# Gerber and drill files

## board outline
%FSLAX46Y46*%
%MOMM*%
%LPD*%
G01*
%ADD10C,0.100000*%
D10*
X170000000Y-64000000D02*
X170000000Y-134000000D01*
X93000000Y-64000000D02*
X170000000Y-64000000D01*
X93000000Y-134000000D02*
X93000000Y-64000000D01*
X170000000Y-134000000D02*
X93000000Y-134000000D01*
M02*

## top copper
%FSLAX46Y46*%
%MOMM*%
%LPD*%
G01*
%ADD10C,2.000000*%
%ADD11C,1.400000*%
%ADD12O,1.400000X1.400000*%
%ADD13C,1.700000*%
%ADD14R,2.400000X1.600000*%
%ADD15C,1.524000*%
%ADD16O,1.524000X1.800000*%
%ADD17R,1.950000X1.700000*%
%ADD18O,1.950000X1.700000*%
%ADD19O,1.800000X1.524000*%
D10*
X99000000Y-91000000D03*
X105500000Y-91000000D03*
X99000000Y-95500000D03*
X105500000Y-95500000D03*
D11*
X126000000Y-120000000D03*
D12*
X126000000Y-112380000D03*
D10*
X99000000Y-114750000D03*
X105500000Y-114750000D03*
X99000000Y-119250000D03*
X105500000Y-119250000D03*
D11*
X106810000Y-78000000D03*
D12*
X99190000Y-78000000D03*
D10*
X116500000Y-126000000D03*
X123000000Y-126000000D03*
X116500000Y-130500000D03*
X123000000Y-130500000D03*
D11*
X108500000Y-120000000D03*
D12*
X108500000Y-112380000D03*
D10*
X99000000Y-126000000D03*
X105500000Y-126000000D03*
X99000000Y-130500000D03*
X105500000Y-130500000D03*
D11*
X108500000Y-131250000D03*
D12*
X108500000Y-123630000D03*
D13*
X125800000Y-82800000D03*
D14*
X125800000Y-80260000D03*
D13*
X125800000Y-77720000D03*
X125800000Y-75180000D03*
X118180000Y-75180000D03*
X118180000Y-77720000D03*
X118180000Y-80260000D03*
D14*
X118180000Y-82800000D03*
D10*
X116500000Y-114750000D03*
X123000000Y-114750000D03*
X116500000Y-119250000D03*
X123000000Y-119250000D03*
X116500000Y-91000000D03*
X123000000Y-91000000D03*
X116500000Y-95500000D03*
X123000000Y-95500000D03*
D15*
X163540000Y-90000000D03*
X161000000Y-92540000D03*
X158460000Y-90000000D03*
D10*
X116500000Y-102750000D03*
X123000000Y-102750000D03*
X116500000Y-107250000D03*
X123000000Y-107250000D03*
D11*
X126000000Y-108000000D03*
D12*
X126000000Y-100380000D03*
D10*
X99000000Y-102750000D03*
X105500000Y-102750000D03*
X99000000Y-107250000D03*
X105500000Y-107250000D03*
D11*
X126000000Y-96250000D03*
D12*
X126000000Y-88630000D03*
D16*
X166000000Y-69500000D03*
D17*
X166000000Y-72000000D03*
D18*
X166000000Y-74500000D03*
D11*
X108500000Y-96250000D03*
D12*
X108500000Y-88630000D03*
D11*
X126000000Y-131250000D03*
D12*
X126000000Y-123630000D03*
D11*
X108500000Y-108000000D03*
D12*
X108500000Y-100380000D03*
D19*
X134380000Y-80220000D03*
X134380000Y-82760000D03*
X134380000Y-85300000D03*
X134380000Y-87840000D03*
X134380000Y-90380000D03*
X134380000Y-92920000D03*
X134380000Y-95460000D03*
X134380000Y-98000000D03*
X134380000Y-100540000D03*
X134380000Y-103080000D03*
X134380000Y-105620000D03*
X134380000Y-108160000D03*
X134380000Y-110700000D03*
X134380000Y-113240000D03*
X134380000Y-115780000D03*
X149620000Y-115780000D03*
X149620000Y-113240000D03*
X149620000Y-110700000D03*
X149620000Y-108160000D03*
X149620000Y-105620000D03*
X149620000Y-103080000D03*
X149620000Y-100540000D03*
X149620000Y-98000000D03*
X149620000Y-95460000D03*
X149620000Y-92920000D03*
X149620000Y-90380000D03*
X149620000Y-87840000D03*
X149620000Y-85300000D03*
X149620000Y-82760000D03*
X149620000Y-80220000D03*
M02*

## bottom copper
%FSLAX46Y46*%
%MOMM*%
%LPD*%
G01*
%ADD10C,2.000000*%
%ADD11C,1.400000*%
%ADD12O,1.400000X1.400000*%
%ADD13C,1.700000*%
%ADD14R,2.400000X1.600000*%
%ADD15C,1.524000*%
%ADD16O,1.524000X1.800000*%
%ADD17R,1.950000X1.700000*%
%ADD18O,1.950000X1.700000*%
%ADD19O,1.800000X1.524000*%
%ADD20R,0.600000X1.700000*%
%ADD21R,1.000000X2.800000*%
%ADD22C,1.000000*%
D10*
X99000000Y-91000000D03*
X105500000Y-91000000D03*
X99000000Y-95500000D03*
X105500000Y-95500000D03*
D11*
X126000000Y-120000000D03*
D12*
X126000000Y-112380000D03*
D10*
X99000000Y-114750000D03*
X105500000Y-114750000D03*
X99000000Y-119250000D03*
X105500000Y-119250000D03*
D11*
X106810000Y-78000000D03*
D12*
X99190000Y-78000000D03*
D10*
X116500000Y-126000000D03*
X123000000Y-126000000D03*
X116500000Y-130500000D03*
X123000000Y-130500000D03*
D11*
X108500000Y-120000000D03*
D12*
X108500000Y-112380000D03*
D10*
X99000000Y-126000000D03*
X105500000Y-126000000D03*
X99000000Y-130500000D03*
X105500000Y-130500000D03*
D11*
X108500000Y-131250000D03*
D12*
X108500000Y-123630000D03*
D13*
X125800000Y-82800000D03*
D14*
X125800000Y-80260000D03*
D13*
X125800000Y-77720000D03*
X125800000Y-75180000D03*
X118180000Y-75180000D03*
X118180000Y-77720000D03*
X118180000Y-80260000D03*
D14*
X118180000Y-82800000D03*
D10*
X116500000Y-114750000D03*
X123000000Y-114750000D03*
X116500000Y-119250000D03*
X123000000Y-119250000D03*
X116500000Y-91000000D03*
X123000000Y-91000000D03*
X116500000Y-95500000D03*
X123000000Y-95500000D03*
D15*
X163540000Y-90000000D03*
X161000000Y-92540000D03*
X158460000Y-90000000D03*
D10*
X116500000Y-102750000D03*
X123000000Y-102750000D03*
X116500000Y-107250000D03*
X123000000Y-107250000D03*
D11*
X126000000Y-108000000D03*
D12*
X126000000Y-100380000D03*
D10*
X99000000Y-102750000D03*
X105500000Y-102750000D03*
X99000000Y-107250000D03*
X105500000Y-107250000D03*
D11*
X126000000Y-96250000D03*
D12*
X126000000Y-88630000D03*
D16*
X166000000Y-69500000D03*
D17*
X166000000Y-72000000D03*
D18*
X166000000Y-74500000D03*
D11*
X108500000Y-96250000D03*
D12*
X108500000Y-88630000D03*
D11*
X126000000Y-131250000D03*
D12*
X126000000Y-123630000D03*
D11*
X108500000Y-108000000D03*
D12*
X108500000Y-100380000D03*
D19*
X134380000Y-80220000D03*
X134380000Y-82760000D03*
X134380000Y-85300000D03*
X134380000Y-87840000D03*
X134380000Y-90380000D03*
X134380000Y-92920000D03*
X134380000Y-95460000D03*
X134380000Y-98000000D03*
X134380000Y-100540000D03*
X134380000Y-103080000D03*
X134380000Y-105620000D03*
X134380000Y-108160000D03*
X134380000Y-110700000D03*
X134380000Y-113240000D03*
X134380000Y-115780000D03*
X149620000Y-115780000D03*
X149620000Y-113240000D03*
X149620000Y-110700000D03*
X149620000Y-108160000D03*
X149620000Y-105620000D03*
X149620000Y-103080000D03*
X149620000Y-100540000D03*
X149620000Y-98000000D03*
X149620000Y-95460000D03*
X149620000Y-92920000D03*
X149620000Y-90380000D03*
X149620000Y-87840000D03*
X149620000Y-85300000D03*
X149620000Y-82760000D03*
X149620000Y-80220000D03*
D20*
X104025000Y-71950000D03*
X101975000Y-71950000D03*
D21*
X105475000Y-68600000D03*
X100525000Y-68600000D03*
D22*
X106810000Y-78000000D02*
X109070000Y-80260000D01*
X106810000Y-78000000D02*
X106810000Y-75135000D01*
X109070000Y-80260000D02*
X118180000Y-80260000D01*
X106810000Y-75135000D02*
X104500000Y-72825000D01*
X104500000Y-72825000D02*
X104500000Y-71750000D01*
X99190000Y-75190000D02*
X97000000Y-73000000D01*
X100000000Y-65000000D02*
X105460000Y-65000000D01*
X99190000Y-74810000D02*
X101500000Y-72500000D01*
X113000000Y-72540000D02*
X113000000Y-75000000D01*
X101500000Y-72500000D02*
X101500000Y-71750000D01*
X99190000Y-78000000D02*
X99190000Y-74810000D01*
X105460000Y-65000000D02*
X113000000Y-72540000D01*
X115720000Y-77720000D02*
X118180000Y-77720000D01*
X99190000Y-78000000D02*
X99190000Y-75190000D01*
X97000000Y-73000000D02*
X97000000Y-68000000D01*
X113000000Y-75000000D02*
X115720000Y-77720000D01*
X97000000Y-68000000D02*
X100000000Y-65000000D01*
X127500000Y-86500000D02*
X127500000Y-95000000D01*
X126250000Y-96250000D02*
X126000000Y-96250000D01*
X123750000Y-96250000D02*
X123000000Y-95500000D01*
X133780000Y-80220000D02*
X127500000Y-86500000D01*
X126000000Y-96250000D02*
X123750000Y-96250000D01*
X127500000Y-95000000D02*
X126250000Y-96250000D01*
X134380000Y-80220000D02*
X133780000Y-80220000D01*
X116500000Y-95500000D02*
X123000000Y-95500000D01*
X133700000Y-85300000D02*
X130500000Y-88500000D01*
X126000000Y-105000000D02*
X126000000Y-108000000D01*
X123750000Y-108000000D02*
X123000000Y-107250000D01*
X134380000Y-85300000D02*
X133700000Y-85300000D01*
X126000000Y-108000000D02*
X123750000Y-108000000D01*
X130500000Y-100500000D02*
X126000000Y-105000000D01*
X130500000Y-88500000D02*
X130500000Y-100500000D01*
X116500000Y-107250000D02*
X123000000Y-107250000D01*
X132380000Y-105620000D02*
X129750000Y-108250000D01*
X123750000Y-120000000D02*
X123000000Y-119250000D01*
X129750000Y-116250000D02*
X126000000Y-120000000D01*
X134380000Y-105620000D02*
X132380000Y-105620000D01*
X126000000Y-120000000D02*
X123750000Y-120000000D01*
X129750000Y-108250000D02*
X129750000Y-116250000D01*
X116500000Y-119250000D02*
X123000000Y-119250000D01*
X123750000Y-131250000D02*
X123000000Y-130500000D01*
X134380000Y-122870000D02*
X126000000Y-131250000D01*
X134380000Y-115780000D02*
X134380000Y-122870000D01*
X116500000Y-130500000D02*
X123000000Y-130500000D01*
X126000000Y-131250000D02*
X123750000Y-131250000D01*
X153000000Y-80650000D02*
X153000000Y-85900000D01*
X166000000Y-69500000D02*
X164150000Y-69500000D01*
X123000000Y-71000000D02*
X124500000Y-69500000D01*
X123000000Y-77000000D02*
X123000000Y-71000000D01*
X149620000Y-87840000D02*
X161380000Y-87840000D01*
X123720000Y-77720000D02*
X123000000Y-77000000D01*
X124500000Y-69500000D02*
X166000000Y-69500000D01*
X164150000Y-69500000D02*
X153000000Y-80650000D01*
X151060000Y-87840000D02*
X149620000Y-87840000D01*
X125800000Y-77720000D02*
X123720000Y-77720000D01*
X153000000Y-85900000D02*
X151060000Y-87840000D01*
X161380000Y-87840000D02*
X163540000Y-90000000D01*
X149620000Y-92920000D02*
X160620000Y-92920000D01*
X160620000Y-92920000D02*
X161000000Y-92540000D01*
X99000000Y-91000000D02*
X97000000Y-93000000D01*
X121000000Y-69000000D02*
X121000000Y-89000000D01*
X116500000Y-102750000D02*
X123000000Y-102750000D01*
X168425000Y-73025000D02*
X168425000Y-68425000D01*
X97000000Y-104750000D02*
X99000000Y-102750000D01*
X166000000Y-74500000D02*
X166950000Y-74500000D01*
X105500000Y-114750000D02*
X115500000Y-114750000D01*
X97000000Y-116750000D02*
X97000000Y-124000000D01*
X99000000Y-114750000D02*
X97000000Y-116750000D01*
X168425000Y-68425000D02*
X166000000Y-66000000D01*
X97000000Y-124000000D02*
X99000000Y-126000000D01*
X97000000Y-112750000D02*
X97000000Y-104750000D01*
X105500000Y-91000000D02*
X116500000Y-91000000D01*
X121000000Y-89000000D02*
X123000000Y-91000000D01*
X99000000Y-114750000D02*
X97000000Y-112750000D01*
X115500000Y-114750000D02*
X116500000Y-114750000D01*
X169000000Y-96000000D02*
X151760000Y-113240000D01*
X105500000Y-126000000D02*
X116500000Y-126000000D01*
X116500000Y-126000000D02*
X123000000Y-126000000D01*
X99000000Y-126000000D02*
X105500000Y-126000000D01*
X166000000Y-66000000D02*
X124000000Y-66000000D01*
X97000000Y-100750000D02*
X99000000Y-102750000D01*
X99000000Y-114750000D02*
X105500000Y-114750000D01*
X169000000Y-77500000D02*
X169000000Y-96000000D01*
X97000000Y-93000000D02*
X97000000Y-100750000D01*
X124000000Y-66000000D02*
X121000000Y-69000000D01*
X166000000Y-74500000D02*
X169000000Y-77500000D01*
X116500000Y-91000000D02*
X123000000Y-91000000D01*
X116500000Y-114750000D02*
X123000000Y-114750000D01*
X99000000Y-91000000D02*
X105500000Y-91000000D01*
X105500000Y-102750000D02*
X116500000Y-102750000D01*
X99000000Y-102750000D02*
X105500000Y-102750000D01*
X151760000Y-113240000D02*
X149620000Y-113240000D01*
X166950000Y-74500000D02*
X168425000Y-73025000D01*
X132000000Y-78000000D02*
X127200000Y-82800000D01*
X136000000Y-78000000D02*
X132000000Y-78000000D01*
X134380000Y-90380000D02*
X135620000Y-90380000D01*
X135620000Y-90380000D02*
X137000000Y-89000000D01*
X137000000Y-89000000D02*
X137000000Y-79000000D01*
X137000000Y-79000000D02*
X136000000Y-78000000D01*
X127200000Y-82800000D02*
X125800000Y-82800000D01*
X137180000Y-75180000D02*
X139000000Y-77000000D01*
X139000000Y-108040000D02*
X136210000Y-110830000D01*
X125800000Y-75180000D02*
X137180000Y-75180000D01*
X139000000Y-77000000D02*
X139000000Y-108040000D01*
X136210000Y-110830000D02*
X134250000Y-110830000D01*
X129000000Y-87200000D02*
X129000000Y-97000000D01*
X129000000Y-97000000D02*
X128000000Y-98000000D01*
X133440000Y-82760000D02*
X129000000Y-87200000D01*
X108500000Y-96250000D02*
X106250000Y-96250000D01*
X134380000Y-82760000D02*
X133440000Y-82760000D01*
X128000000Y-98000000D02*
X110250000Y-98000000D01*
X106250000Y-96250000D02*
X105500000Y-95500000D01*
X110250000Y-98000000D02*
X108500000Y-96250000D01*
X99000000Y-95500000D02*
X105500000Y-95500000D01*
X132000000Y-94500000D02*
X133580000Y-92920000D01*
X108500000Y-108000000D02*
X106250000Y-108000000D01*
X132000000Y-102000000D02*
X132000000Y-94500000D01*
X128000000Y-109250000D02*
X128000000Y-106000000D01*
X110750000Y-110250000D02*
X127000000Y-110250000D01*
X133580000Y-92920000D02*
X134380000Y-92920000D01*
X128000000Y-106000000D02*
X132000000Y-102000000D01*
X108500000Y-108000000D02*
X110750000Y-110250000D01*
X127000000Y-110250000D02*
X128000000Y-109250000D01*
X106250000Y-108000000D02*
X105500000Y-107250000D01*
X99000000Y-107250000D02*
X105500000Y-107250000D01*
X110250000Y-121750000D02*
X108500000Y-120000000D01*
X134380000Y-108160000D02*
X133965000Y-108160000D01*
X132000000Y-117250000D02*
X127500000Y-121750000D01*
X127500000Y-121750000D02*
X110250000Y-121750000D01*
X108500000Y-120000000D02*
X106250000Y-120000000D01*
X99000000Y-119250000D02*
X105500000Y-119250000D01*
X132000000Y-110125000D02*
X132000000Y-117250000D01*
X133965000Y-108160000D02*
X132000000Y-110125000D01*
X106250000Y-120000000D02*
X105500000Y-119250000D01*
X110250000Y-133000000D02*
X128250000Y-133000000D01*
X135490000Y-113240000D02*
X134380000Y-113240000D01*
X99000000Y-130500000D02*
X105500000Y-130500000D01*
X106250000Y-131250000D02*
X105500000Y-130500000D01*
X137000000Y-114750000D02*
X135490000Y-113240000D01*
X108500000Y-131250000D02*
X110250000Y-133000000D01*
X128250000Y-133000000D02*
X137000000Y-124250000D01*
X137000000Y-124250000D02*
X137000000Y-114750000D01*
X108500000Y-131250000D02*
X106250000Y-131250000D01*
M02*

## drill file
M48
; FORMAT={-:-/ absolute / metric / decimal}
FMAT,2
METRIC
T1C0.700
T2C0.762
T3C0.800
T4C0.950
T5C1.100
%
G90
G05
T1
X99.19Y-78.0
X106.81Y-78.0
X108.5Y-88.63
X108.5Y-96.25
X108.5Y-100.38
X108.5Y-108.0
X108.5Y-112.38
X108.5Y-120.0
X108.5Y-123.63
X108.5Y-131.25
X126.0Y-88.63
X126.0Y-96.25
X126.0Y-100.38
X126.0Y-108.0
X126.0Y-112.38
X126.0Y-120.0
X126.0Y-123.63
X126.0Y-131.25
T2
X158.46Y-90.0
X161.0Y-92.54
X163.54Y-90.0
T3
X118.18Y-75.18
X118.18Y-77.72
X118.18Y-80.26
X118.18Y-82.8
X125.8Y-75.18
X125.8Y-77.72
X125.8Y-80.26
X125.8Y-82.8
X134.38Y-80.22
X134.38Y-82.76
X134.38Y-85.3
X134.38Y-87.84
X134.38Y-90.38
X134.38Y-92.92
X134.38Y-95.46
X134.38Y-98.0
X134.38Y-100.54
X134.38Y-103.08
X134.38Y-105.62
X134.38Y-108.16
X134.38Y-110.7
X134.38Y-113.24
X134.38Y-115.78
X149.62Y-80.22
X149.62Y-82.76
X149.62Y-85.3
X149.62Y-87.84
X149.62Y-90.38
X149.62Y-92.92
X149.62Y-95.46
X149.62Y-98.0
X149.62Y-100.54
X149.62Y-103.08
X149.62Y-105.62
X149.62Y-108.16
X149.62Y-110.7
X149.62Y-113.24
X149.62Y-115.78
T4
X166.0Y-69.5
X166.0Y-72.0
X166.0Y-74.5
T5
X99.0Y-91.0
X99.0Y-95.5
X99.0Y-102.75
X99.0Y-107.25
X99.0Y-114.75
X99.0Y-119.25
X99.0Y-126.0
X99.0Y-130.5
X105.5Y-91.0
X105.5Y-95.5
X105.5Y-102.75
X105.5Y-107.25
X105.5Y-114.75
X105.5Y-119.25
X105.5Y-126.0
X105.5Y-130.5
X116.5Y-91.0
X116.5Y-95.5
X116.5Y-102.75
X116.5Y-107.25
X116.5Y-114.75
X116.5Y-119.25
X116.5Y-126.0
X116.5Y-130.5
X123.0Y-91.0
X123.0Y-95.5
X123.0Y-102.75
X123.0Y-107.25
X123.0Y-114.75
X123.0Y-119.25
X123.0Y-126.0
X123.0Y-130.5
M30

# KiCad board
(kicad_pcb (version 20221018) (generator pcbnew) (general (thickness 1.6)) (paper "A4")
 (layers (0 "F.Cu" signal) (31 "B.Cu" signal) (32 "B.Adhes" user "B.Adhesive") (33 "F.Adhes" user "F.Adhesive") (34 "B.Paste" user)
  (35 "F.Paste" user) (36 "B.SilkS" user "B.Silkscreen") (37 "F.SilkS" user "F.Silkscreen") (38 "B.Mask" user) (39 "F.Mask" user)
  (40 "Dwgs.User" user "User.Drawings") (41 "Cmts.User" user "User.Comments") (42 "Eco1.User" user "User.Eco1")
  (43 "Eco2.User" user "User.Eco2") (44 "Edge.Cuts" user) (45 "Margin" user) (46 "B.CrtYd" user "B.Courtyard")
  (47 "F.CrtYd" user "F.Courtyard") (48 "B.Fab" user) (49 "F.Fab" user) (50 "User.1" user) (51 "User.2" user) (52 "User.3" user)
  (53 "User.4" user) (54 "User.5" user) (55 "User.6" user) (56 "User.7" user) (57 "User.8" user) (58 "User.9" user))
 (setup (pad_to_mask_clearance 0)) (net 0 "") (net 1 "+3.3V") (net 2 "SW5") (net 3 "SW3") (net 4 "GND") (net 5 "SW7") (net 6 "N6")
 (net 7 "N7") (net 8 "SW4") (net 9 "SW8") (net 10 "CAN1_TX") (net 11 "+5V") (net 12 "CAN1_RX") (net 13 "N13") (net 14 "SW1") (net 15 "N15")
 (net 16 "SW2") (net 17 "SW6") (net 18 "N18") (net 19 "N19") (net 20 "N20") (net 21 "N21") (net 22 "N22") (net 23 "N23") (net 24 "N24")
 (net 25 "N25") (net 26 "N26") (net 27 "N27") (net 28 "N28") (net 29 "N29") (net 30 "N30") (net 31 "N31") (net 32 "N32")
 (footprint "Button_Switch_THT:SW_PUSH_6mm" (layer "F.Cu") (at 99 91)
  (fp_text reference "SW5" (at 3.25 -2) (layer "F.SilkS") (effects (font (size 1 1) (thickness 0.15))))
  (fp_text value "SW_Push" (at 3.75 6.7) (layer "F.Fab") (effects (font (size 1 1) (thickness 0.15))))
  (pad "1" thru_hole circle (at 0 0 90) (size 2 2) (drill 1.1) (layers "*.Cu" "*.Mask") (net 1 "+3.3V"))
  (pad "1" thru_hole circle (at 6.5 0 90) (size 2 2) (drill 1.1) (layers "*.Cu" "*.Mask") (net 1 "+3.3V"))
  (pad "2" thru_hole circle (at 0 4.5 90) (size 2 2) (drill 1.1) (layers "*.Cu" "*.Mask") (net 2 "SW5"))
  (pad "2" thru_hole circle (at 6.5 4.5 90) (size 2 2) (drill 1.1) (layers "*.Cu" "*.Mask") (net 2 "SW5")))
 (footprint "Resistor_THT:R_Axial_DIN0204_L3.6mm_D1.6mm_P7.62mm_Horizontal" (layer "F.Cu") (at 126 120 90)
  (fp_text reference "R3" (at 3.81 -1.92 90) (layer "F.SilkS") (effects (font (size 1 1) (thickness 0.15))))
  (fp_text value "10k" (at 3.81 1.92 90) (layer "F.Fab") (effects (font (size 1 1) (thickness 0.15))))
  (pad "1" thru_hole circle (at 0 0 90) (size 1.4 1.4) (drill 0.7) (layers "*.Cu" "*.Mask") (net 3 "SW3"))
  (pad "2" thru_hole oval (at 7.62 0 90) (size 1.4 1.4) (drill 0.7) (layers "*.Cu" "*.Mask") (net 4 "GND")))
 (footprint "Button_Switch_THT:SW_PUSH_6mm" (layer "F.Cu") (at 99 114.75)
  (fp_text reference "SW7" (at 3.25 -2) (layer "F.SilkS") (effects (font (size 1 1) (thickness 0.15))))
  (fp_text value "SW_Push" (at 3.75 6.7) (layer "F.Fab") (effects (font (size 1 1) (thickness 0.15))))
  (pad "1" thru_hole circle (at 0 0 90) (size 2 2) (drill 1.1) (layers "*.Cu" "*.Mask") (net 1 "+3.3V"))
  (pad "1" thru_hole circle (at 6.5 0 90) (size 2 2) (drill 1.1) (layers "*.Cu" "*.Mask") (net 1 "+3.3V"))
  (pad "2" thru_hole circle (at 0 4.5 90) (size 2 2) (drill 1.1) (layers "*.Cu" "*.Mask") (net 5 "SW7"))
  (pad "2" thru_hole circle (at 6.5 4.5 90) (size 2 2) (drill 1.1) (layers "*.Cu" "*.Mask") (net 5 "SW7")))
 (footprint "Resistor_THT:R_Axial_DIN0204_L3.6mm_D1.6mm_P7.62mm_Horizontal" (layer "F.Cu") (at 106.81 78 180)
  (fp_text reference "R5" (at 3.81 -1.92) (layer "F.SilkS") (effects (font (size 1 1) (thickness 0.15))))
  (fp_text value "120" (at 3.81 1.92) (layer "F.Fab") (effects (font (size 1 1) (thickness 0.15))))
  (pad "1" thru_hole circle (at 0 0 180) (size 1.4 1.4) (drill 0.7) (layers "*.Cu" "*.Mask") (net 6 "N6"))
  (pad "2" thru_hole oval (at 7.62 0 180) (size 1.4 1.4) (drill 0.7) (layers "*.Cu" "*.Mask") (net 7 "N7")))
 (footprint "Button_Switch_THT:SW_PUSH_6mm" (layer "F.Cu") (at 116.5 126)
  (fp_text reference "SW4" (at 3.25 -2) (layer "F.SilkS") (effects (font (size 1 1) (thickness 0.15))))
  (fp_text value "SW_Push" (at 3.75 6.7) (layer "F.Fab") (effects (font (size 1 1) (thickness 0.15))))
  (pad "1" thru_hole circle (at 0 0 90) (size 2 2) (drill 1.1) (layers "*.Cu" "*.Mask") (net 1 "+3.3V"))
  (pad "1" thru_hole circle (at 6.5 0 90) (size 2 2) (drill 1.1) (layers "*.Cu" "*.Mask") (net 1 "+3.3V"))
  (pad "2" thru_hole circle (at 0 4.5 90) (size 2 2) (drill 1.1) (layers "*.Cu" "*.Mask") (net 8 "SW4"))
  (pad "2" thru_hole circle (at 6.5 4.5 90) (size 2 2) (drill 1.1) (layers "*.Cu" "*.Mask") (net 8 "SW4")))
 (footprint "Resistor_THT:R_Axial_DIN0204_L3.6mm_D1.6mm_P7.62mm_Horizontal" (layer "F.Cu") (at 108.5 120 90)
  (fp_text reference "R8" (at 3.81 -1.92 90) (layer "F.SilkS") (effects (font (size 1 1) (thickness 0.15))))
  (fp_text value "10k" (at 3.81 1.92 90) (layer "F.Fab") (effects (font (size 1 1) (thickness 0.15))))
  (pad "1" thru_hole circle (at 0 0 90) (size 1.4 1.4) (drill 0.7) (layers "*.Cu" "*.Mask") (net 5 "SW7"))
  (pad "2" thru_hole oval (at 7.62 0 90) (size 1.4 1.4) (drill 0.7) (layers "*.Cu" "*.Mask") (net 4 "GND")))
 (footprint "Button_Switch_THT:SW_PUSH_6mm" (layer "F.Cu") (at 99 126)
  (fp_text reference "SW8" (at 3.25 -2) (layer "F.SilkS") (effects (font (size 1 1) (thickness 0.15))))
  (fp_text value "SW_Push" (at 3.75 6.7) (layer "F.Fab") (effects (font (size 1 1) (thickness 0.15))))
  (pad "1" thru_hole circle (at 0 0 90) (size 2 2) (drill 1.1) (layers "*.Cu" "*.Mask") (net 1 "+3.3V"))
  (pad "1" thru_hole circle (at 6.5 0 90) (size 2 2) (drill 1.1) (layers "*.Cu" "*.Mask") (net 1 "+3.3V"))
  (pad "2" thru_hole circle (at 0 4.5 90) (size 2 2) (drill 1.1) (layers "*.Cu" "*.Mask") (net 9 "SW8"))
  (pad "2" thru_hole circle (at 6.5 4.5 90) (size 2 2) (drill 1.1) (layers "*.Cu" "*.Mask") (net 9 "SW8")))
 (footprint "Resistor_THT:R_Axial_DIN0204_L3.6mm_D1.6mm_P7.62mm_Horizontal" (layer "F.Cu") (at 108.5 131.25 90)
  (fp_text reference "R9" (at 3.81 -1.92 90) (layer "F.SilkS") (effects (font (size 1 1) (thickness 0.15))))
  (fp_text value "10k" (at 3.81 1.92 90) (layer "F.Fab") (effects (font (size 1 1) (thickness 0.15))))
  (pad "1" thru_hole circle (at 0 0 90) (size 1.4 1.4) (drill 0.7) (layers "*.Cu" "*.Mask") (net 9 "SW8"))
  (pad "2" thru_hole oval (at 7.62 0 90) (size 1.4 1.4) (drill 0.7) (layers "*.Cu" "*.Mask") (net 4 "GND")))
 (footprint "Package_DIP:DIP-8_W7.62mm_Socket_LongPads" (layer "F.Cu") (at 125.8 82.8 180)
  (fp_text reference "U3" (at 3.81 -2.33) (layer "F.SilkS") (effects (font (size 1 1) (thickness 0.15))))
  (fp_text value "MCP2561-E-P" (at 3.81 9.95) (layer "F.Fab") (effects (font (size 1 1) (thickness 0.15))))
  (pad "1" thru_hole circle (at 0 0 180) (size 1.7 1.7) (drill 0.8) (layers "*.Cu" "*.Mask") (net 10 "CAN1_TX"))
  (pad "2" thru_hole rect (at 0 2.54 180) (size 2.4 1.6) (drill 0.8) (layers "*.Cu" "*.Mask") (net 4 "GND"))
  (pad "3" thru_hole circle (at 0 5.08 180) (size 1.7 1.7) (drill 0.8) (layers "*.Cu" "*.Mask") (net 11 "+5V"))
  (pad "4" thru_hole circle (at 0 7.62 180) (size 1.7 1.7) (drill 0.8) (layers "*.Cu" "*.Mask") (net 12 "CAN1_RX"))
  (pad "5" thru_hole circle (at 7.62 7.62 180) (size 1.7 1.7) (drill 0.8) (layers "*.Cu" "*.Mask") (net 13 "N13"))
  (pad "6" thru_hole circle (at 7.62 5.08 180) (size 1.7 1.7) (drill 0.8) (layers "*.Cu" "*.Mask") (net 7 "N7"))
  (pad "7" thru_hole circle (at 7.62 2.54 180) (size 1.7 1.7) (drill 0.8) (layers "*.Cu" "*.Mask") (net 6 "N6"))
  (pad "8" thru_hole rect (at 7.62 0 180) (size 2.4 1.6) (drill 0.8) (layers "*.Cu" "*.Mask") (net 4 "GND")))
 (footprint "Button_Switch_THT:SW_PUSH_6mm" (layer "F.Cu") (at 116.5 114.75)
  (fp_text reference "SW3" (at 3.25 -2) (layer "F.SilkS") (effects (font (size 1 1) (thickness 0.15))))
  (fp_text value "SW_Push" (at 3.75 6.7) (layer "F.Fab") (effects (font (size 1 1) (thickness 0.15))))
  (pad "1" thru_hole circle (at 0 0 90) (size 2 2) (drill 1.1) (layers "*.Cu" "*.Mask") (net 1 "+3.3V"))
  (pad "1" thru_hole circle (at 6.5 0 90) (size 2 2) (drill 1.1) (layers "*.Cu" "*.Mask") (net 1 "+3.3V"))
  (pad "2" thru_hole circle (at 0 4.5 90) (size 2 2) (drill 1.1) (layers "*.Cu" "*.Mask") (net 3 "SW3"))
  (pad "2" thru_hole circle (at 6.5 4.5 90) (size 2 2) (drill 1.1) (layers "*.Cu" "*.Mask") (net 3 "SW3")))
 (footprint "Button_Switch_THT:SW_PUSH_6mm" (layer "F.Cu") (at 116.5 91)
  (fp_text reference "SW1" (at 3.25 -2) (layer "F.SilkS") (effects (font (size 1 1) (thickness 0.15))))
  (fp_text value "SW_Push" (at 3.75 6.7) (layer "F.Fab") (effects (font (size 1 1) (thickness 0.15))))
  (pad "1" thru_hole circle (at 0 0 90) (size 2 2) (drill 1.1) (layers "*.Cu" "*.Mask") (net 1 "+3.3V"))
  (pad "1" thru_hole circle (at 6.5 0 90) (size 2 2) (drill 1.1) (layers "*.Cu" "*.Mask") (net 1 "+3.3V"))
  (pad "2" thru_hole circle (at 0 4.5 90) (size 2 2) (drill 1.1) (layers "*.Cu" "*.Mask") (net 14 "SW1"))
  (pad "2" thru_hole circle (at 6.5 4.5 90) (size 2 2) (drill 1.1) (layers "*.Cu" "*.Mask") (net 14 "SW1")))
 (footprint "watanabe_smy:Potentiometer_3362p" (layer "F.Cu") (at 161 90 180)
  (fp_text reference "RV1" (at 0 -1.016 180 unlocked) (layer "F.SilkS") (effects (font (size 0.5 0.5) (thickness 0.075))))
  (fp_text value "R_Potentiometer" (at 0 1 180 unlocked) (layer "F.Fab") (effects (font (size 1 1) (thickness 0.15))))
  (pad "1" thru_hole circle (at -2.54 0 180) (size 1.524 1.524) (drill 0.762) (layers "*.Cu" "*.Mask") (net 11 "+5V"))
  (pad "2" thru_hole circle (at 0 -2.54 180) (size 1.524 1.524) (drill 0.762) (layers "*.Cu" "*.Mask") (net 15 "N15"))
  (pad "3" thru_hole circle (at 2.54 0 180) (size 1.524 1.524) (drill 0.762) (layers "*.Cu" "*.Mask") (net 4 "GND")))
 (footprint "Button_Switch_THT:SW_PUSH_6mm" (layer "F.Cu") (at 116.5 102.75)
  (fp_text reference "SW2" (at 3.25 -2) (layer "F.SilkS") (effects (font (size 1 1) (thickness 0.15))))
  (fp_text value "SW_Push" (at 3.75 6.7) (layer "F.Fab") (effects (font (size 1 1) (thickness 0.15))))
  (pad "1" thru_hole circle (at 0 0 90) (size 2 2) (drill 1.1) (layers "*.Cu" "*.Mask") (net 1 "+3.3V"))
  (pad "1" thru_hole circle (at 6.5 0 90) (size 2 2) (drill 1.1) (layers "*.Cu" "*.Mask") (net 1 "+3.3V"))
  (pad "2" thru_hole circle (at 0 4.5 90) (size 2 2) (drill 1.1) (layers "*.Cu" "*.Mask") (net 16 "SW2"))
  (pad "2" thru_hole circle (at 6.5 4.5 90) (size 2 2) (drill 1.1) (layers "*.Cu" "*.Mask") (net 16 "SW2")))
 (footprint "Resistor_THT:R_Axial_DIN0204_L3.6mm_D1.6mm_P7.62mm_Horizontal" (layer "F.Cu") (at 126 108 90)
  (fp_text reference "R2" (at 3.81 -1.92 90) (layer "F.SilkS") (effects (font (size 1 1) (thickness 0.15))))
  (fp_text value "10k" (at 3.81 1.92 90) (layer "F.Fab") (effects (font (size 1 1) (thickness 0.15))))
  (pad "1" thru_hole circle (at 0 0 90) (size 1.4 1.4) (drill 0.7) (layers "*.Cu" "*.Mask") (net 16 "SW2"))
  (pad "2" thru_hole oval (at 7.62 0 90) (size 1.4 1.4) (drill 0.7) (layers "*.Cu" "*.Mask") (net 4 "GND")))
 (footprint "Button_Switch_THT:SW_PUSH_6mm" (layer "F.Cu") (at 99 102.75)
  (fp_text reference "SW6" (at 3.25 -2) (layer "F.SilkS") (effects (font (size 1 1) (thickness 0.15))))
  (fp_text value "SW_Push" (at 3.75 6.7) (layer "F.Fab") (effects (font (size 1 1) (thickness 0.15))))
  (pad "1" thru_hole circle (at 0 0 90) (size 2 2) (drill 1.1) (layers "*.Cu" "*.Mask") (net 1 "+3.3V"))
  (pad "1" thru_hole circle (at 6.5 0 90) (size 2 2) (drill 1.1) (layers "*.Cu" "*.Mask") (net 1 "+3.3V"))
  (pad "2" thru_hole circle (at 0 4.5 90) (size 2 2) (drill 1.1) (layers "*.Cu" "*.Mask") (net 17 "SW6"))
  (pad "2" thru_hole circle (at 6.5 4.5 90) (size 2 2) (drill 1.1) (layers "*.Cu" "*.Mask") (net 17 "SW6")))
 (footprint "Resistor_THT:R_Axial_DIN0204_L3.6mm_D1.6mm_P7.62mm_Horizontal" (layer "F.Cu") (at 126 96.25 90)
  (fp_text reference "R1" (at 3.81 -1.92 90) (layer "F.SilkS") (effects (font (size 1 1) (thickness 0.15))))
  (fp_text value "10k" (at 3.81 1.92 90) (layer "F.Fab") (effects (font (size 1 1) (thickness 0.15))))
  (pad "1" thru_hole circle (at 0 0 90) (size 1.4 1.4) (drill 0.7) (layers "*.Cu" "*.Mask") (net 14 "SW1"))
  (pad "2" thru_hole oval (at 7.62 0 90) (size 1.4 1.4) (drill 0.7) (layers "*.Cu" "*.Mask") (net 4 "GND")))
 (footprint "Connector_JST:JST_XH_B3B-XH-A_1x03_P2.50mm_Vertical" (layer "F.Cu") (at 166 69.5 -90)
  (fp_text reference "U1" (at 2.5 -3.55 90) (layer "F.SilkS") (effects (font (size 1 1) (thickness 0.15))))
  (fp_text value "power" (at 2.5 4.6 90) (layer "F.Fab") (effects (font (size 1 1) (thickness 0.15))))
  (pad "1" thru_hole oval (at 0 0 270) (size 1.8 1.524) (drill 0.95) (layers "*.Cu" "*.Mask") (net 11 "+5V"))
  (pad "2" thru_hole rect (at 2.5 0 270) (size 1.7 1.95) (drill 0.95) (layers "*.Cu" "*.Mask") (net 4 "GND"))
  (pad "3" thru_hole oval (at 5 0 270) (size 1.7 1.95) (drill 0.95) (layers "*.Cu" "*.Mask") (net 1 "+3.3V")))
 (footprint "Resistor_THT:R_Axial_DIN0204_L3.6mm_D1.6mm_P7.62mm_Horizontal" (layer "F.Cu") (at 108.5 96.25 90)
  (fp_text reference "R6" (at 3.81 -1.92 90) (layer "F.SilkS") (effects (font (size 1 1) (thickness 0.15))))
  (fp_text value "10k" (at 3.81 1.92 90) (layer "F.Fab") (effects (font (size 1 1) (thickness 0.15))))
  (pad "1" thru_hole circle (at 0 0 90) (size 1.4 1.4) (drill 0.7) (layers "*.Cu" "*.Mask") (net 2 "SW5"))
  (pad "2" thru_hole oval (at 7.62 0 90) (size 1.4 1.4) (drill 0.7) (layers "*.Cu" "*.Mask") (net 4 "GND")))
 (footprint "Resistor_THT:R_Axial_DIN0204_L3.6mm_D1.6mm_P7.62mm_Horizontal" (layer "F.Cu") (at 126 131.25 90)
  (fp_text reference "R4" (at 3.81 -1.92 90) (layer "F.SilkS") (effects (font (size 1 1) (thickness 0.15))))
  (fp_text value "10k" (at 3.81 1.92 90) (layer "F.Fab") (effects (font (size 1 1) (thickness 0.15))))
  (pad "1" thru_hole circle (at 0 0 90) (size 1.4 1.4) (drill 0.7) (layers "*.Cu" "*.Mask") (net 8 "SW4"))
  (pad "2" thru_hole oval (at 7.62 0 90) (size 1.4 1.4) (drill 0.7) (layers "*.Cu" "*.Mask") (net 4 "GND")))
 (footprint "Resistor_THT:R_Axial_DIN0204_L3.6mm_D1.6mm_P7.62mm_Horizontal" (layer "F.Cu") (at 108.5 108 90)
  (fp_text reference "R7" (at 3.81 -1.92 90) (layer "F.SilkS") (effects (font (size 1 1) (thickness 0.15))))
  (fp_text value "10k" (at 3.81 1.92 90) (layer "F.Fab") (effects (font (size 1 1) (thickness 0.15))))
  (pad "1" thru_hole circle (at 0 0 90) (size 1.4 1.4) (drill 0.7) (layers "*.Cu" "*.Mask") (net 17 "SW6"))
  (pad "2" thru_hole oval (at 7.62 0 90) (size 1.4 1.4) (drill 0.7) (layers "*.Cu" "*.Mask") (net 4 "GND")))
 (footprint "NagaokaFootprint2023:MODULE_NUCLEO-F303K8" (layer "F.Cu") (at 142 98)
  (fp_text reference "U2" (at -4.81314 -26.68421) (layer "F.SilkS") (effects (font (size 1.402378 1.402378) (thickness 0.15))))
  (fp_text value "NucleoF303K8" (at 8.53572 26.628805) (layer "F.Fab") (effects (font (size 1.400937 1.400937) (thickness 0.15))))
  (pad "1" thru_hole oval (at -7.62 -17.78) (size 1.8 1.524) (drill 0.8) (layers "*.Cu" "*.Mask") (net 14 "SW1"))
  (pad "2" thru_hole oval (at -7.62 -15.24) (size 1.8 1.524) (drill 0.8) (layers "*.Cu" "*.Mask") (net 2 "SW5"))
  (pad "3" thru_hole oval (at -7.62 -12.7) (size 1.8 1.524) (drill 0.8) (layers "*.Cu" "*.Mask") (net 16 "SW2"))
  (pad "4" thru_hole oval (at -7.62 -10.16) (size 1.8 1.524) (drill 0.8) (layers "*.Cu" "*.Mask") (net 4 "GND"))
  (pad "5" thru_hole oval (at -7.62 -7.62) (size 1.8 1.524) (drill 0.8) (layers "*.Cu" "*.Mask") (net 10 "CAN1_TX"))
  (pad "6" thru_hole oval (at -7.62 -5.08) (size 1.8 1.524) (drill 0.8) (layers "*.Cu" "*.Mask") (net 17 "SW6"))
  (pad "7" thru_hole oval (at -7.62 -2.54) (size 1.8 1.524) (drill 0.8) (layers "*.Cu" "*.Mask") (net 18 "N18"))
  (pad "8" thru_hole oval (at -7.62 0) (size 1.8 1.524) (drill 0.8) (layers "*.Cu" "*.Mask") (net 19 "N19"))
  (pad "9" thru_hole oval (at -7.62 2.54) (size 1.8 1.524) (drill 0.8) (layers "*.Cu" "*.Mask") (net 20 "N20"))
  (pad "10" thru_hole oval (at -7.62 5.08) (size 1.8 1.524) (drill 0.8) (layers "*.Cu" "*.Mask") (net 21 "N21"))
  (pad "11" thru_hole oval (at -7.62 7.62) (size 1.8 1.524) (drill 0.8) (layers "*.Cu" "*.Mask") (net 3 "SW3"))
  (pad "12" thru_hole oval (at -7.62 10.16) (size 1.8 1.524) (drill 0.8) (layers "*.Cu" "*.Mask") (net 5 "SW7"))
  (pad "13" thru_hole oval (at -7.62 12.7) (size 1.8 1.524) (drill 0.8) (layers "*.Cu" "*.Mask") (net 12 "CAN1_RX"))
  (pad "14" thru_hole oval (at -7.62 15.24) (size 1.8 1.524) (drill 0.8) (layers "*.Cu" "*.Mask") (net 9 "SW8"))
  (pad "15" thru_hole oval (at -7.62 17.78) (size 1.8 1.524) (drill 0.8) (layers "*.Cu" "*.Mask") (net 8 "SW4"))
  (pad "16" thru_hole oval (at 7.62 17.78) (size 1.8 1.524) (drill 0.8) (layers "*.Cu" "*.Mask") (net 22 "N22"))
  (pad "17" thru_hole oval (at 7.62 15.24) (size 1.8 1.524) (drill 0.8) (layers "*.Cu" "*.Mask") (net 1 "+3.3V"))
  (pad "18" thru_hole oval (at 7.62 12.7) (size 1.8 1.524) (drill 0.8) (layers "*.Cu" "*.Mask") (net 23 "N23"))
  (pad "19" thru_hole oval (at 7.62 10.16) (size 1.8 1.524) (drill 0.8) (layers "*.Cu" "*.Mask") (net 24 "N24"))
  (pad "20" thru_hole oval (at 7.62 7.62) (size 1.8 1.524) (drill 0.8) (layers "*.Cu" "*.Mask") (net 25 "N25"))
  (pad "21" thru_hole oval (at 7.62 5.08) (size 1.8 1.524) (drill 0.8) (layers "*.Cu" "*.Mask") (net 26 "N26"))
  (pad "22" thru_hole oval (at 7.62 2.54) (size 1.8 1.524) (drill 0.8) (layers "*.Cu" "*.Mask") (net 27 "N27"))
  (pad "23" thru_hole oval (at 7.62 0) (size 1.8 1.524) (drill 0.8) (layers "*.Cu" "*.Mask") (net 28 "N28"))
  (pad "24" thru_hole oval (at 7.62 -2.54) (size 1.8 1.524) (drill 0.8) (layers "*.Cu" "*.Mask") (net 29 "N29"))
  (pad "25" thru_hole oval (at 7.62 -5.08) (size 1.8 1.524) (drill 0.8) (layers "*.Cu" "*.Mask") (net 15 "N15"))
  (pad "26" thru_hole oval (at 7.62 -7.62) (size 1.8 1.524) (drill 0.8) (layers "*.Cu" "*.Mask") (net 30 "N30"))
  (pad "27" thru_hole oval (at 7.62 -10.16) (size 1.8 1.524) (drill 0.8) (layers "*.Cu" "*.Mask") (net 11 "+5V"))
  (pad "28" thru_hole oval (at 7.62 -12.7) (size 1.8 1.524) (drill 0.8) (layers "*.Cu" "*.Mask") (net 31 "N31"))
  (pad "29" thru_hole oval (at 7.62 -15.24) (size 1.8 1.524) (drill 0.8) (layers "*.Cu" "*.Mask") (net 4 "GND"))
  (pad "30" thru_hole oval (at 7.62 -17.78) (size 1.8 1.524) (drill 0.8) (layers "*.Cu" "*.Mask") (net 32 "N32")))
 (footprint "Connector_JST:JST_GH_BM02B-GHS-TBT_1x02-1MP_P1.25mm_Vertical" (layer "B.Cu") (at 103 70 180)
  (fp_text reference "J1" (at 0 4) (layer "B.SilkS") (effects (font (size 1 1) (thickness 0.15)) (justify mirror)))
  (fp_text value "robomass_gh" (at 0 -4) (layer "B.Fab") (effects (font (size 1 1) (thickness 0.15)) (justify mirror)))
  (pad "1" smd rect (at -1.025 -1.95 180) (size 0.6 1.7) (layers "B.Cu" "B.Paste" "B.Mask") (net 6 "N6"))
  (pad "2" smd rect (at 1.025 -1.95 180) (size 0.6 1.7) (layers "B.Cu" "B.Paste" "B.Mask") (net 7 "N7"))
  (pad "MP" smd rect (at -2.475 1.4 180) (size 1 2.8) (layers "B.Cu" "B.Paste" "B.Mask"))
  (pad "MP" smd rect (at 2.475 1.4 180) (size 1 2.8) (layers "B.Cu" "B.Paste" "B.Mask")))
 (gr_line (start 170 64) (end 170 134) (stroke (width 0.1) (type default)) (layer "Edge.Cuts"))
 (gr_line (start 93 64) (end 170 64) (stroke (width 0.1) (type default)) (layer "Edge.Cuts"))
 (gr_line (start 93 134) (end 93 64) (stroke (width 0.1) (type default)) (layer "Edge.Cuts"))
 (gr_line (start 170 134) (end 93 134) (stroke (width 0.1) (type default)) (layer "Edge.Cuts"))
 (segment (start 106.81 78) (end 109.07 80.26) (width 1) (layer "B.Cu") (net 6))
 (segment (start 106.81 78) (end 106.81 75.135) (width 1) (layer "B.Cu") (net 6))
 (segment (start 109.07 80.26) (end 118.18 80.26) (width 1) (layer "B.Cu") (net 6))
 (segment (start 106.81 75.135) (end 104.5 72.825) (width 1) (layer "B.Cu") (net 6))
 (segment (start 104.5 72.825) (end 104.5 71.75) (width 1) (layer "B.Cu") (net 6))
 (segment (start 99.19 75.19) (end 97 73) (width 1) (layer "B.Cu") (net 7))
 (segment (start 100 65) (end 105.46 65) (width 1) (layer "B.Cu") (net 7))
 (segment (start 99.19 74.81) (end 101.5 72.5) (width 1) (layer "B.Cu") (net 7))
 (segment (start 113 72.54) (end 113 75) (width 1) (layer "B.Cu") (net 7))
 (segment (start 101.5 72.5) (end 101.5 71.75) (width 1) (layer "B.Cu") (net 7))
 (segment (start 99.19 78) (end 99.19 74.81) (width 1) (layer "B.Cu") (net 7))
 (segment (start 105.46 65) (end 113 72.54) (width 1) (layer "B.Cu") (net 7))
 (segment (start 115.72 77.72) (end 118.18 77.72) (width 1) (layer "B.Cu") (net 7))
 (segment (start 99.19 78) (end 99.19 75.19) (width 1) (layer "B.Cu") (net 7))
 (segment (start 97 73) (end 97 68) (width 1) (layer "B.Cu") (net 7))
 (segment (start 113 75) (end 115.72 77.72) (width 1) (layer "B.Cu") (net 7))
 (segment (start 97 68) (end 100 65) (width 1) (layer "B.Cu") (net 7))
 (segment (start 127.5 86.5) (end 127.5 95) (width 1) (layer "B.Cu") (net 14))
 (segment (start 126.25 96.25) (end 126 96.25) (width 1) (layer "B.Cu") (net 14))
 (segment (start 123.75 96.25) (end 123 95.5) (width 1) (layer "B.Cu") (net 14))
 (segment (start 133.78 80.22) (end 127.5 86.5) (width 1) (layer "B.Cu") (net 14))
 (segment (start 126 96.25) (end 123.75 96.25) (width 1) (layer "B.Cu") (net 14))
 (segment (start 127.5 95) (end 126.25 96.25) (width 1) (layer "B.Cu") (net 14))
 (segment (start 134.38 80.22) (end 133.78 80.22) (width 1) (layer "B.Cu") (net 14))
 (segment (start 116.5 95.5) (end 123 95.5) (width 1) (layer "B.Cu") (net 14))
 (segment (start 133.7 85.3) (end 130.5 88.5) (width 1) (layer "B.Cu") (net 16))
 (segment (start 126 105) (end 126 108) (width 1) (layer "B.Cu") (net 16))
 (segment (start 123.75 108) (end 123 107.25) (width 1) (layer "B.Cu") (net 16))
 (segment (start 134.38 85.3) (end 133.7 85.3) (width 1) (layer "B.Cu") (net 16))
 (segment (start 126 108) (end 123.75 108) (width 1) (layer "B.Cu") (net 16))
 (segment (start 130.5 100.5) (end 126 105) (width 1) (layer "B.Cu") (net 16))
 (segment (start 130.5 88.5) (end 130.5 100.5) (width 1) (layer "B.Cu") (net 16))
 (segment (start 116.5 107.25) (end 123 107.25) (width 1) (layer "B.Cu") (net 16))
 (segment (start 132.38 105.62) (end 129.75 108.25) (width 1) (layer "B.Cu") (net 3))
 (segment (start 123.75 120) (end 123 119.25) (width 1) (layer "B.Cu") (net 3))
 (segment (start 129.75 116.25) (end 126 120) (width 1) (layer "B.Cu") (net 3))
 (segment (start 134.38 105.62) (end 132.38 105.62) (width 1) (layer "B.Cu") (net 3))
 (segment (start 126 120) (end 123.75 120) (width 1) (layer "B.Cu") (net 3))
 (segment (start 129.75 108.25) (end 129.75 116.25) (width 1) (layer "B.Cu") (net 3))
 (segment (start 116.5 119.25) (end 123 119.25) (width 1) (layer "B.Cu") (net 3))
 (segment (start 123.75 131.25) (end 123 130.5) (width 1) (layer "B.Cu") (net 8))
 (segment (start 134.38 122.87) (end 126 131.25) (width 1) (layer "B.Cu") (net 8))
 (segment (start 134.38 115.78) (end 134.38 122.87) (width 1) (layer "B.Cu") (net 8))
 (segment (start 116.5 130.5) (end 123 130.5) (width 1) (layer "B.Cu") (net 8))
 (segment (start 126 131.25) (end 123.75 131.25) (width 1) (layer "B.Cu") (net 8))
 (segment (start 153 80.65) (end 153 85.9) (width 1) (layer "B.Cu") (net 11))
 (segment (start 166 69.5) (end 164.15 69.5) (width 1) (layer "B.Cu") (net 11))
 (segment (start 123 71) (end 124.5 69.5) (width 1) (layer "B.Cu") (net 11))
 (segment (start 123 77) (end 123 71) (width 1) (layer "B.Cu") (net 11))
 (segment (start 149.62 87.84) (end 161.38 87.84) (width 1) (layer "B.Cu") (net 11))
 (segment (start 123.72 77.72) (end 123 77) (width 1) (layer "B.Cu") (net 11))
 (segment (start 124.5 69.5) (end 166 69.5) (width 1) (layer "B.Cu") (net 11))
 (segment (start 164.15 69.5) (end 153 80.65) (width 1) (layer "B.Cu") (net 11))
 (segment (start 151.06 87.84) (end 149.62 87.84) (width 1) (layer "B.Cu") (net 11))
 (segment (start 125.8 77.72) (end 123.72 77.72) (width 1) (layer "B.Cu") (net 11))
 (segment (start 153 85.9) (end 151.06 87.84) (width 1) (layer "B.Cu") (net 11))
 (segment (start 161.38 87.84) (end 163.54 90) (width 1) (layer "B.Cu") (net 11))
 (segment (start 149.62 92.92) (end 160.62 92.92) (width 1) (layer "B.Cu") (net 15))
 (segment (start 160.62 92.92) (end 161 92.54) (width 1) (layer "B.Cu") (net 15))
 (segment (start 99 91) (end 97 93) (width 1) (layer "B.Cu") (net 1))
 (segment (start 121 69) (end 121 89) (width 1) (layer "B.Cu") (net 1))
 (segment (start 116.5 102.75) (end 123 102.75) (width 1) (layer "B.Cu") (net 1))
 (segment (start 168.425 73.025) (end 168.425 68.425) (width 1) (layer "B.Cu") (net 1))
 (segment (start 97 104.75) (end 99 102.75) (width 1) (layer "B.Cu") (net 1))
 (segment (start 166 74.5) (end 166.95 74.5) (width 1) (layer "B.Cu") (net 1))
 (segment (start 105.5 114.75) (end 115.5 114.75) (width 1) (layer "B.Cu") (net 1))
 (segment (start 97 116.75) (end 97 124) (width 1) (layer "B.Cu") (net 1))
 (segment (start 99 114.75) (end 97 116.75) (width 1) (layer "B.Cu") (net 1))
 (segment (start 168.425 68.425) (end 166 66) (width 1) (layer "B.Cu") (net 1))
 (segment (start 97 124) (end 99 126) (width 1) (layer "B.Cu") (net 1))
 (segment (start 97 112.75) (end 97 104.75) (width 1) (layer "B.Cu") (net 1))
 (segment (start 105.5 91) (end 116.5 91) (width 1) (layer "B.Cu") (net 1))
 (segment (start 121 89) (end 123 91) (width 1) (layer "B.Cu") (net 1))
 (segment (start 99 114.75) (end 97 112.75) (width 1) (layer "B.Cu") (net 1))
 (segment (start 115.5 114.75) (end 116.5 114.75) (width 1) (layer "B.Cu") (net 1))
 (segment (start 169 96) (end 151.76 113.24) (width 1) (layer "B.Cu") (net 1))
 (segment (start 105.5 126) (end 116.5 126) (width 1) (layer "B.Cu") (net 1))
 (segment (start 116.5 126) (end 123 126) (width 1) (layer "B.Cu") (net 1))
 (segment (start 99 126) (end 105.5 126) (width 1) (layer "B.Cu") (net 1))
 (segment (start 166 66) (end 124 66) (width 1) (layer "B.Cu") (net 1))
 (segment (start 97 100.75) (end 99 102.75) (width 1) (layer "B.Cu") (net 1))
 (segment (start 99 114.75) (end 105.5 114.75) (width 1) (layer "B.Cu") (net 1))
 (segment (start 169 77.5) (end 169 96) (width 1) (layer "B.Cu") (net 1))
 (segment (start 97 93) (end 97 100.75) (width 1) (layer "B.Cu") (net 1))
 (segment (start 124 66) (end 121 69) (width 1) (layer "B.Cu") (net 1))
 (segment (start 166 74.5) (end 169 77.5) (width 1) (layer "B.Cu") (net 1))
 (segment (start 116.5 91) (end 123 91) (width 1) (layer "B.Cu") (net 1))
 (segment (start 116.5 114.75) (end 123 114.75) (width 1) (layer "B.Cu") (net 1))
 (segment (start 99 91) (end 105.5 91) (width 1) (layer "B.Cu") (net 1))
 (segment (start 105.5 102.75) (end 116.5 102.75) (width 1) (layer "B.Cu") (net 1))
 (segment (start 99 102.75) (end 105.5 102.75) (width 1) (layer "B.Cu") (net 1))
 (segment (start 151.76 113.24) (end 149.62 113.24) (width 1) (layer "B.Cu") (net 1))
 (segment (start 166.95 74.5) (end 168.425 73.025) (width 1) (layer "B.Cu") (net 1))
 (segment (start 132 78) (end 127.2 82.8) (width 1) (layer "B.Cu") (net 10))
 (segment (start 136 78) (end 132 78) (width 1) (layer "B.Cu") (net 10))
 (segment (start 134.38 90.38) (end 135.62 90.38) (width 1) (layer "B.Cu") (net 10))
 (segment (start 135.62 90.38) (end 137 89) (width 1) (layer "B.Cu") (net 10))
 (segment (start 137 89) (end 137 79) (width 1) (layer "B.Cu") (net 10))
 (segment (start 137 79) (end 136 78) (width 1) (layer "B.Cu") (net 10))
 (segment (start 127.2 82.8) (end 125.8 82.8) (width 1) (layer "B.Cu") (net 10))
 (segment (start 137.18 75.18) (end 139 77) (width 1) (layer "B.Cu") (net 12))
 (segment (start 139 108.04) (end 136.21 110.83) (width 1) (layer "B.Cu") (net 12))
 (segment (start 125.8 75.18) (end 137.18 75.18) (width 1) (layer "B.Cu") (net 12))
 (segment (start 139 77) (end 139 108.04) (width 1) (layer "B.Cu") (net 12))
 (segment (start 136.21 110.83) (end 134.25 110.83) (width 1) (layer "B.Cu") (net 12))
 (segment (start 129 87.2) (end 129 97) (width 1) (layer "B.Cu") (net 2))
 (segment (start 129 97) (end 128 98) (width 1) (layer "B.Cu") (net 2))
 (segment (start 133.44 82.76) (end 129 87.2) (width 1) (layer "B.Cu") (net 2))
 (segment (start 108.5 96.25) (end 106.25 96.25) (width 1) (layer "B.Cu") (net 2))
 (segment (start 134.38 82.76) (end 133.44 82.76) (width 1) (layer "B.Cu") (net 2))
 (segment (start 128 98) (end 110.25 98) (width 1) (layer "B.Cu") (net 2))
 (segment (start 106.25 96.25) (end 105.5 95.5) (width 1) (layer "B.Cu") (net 2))
 (segment (start 110.25 98) (end 108.5 96.25) (width 1) (layer "B.Cu") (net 2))
 (segment (start 99 95.5) (end 105.5 95.5) (width 1) (layer "B.Cu") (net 2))
 (segment (start 132 94.5) (end 133.58 92.92) (width 1) (layer "B.Cu") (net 17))
 (segment (start 108.5 108) (end 106.25 108) (width 1) (layer "B.Cu") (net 17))
 (segment (start 132 102) (end 132 94.5) (width 1) (layer "B.Cu") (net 17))
 (segment (start 128 109.25) (end 128 106) (width 1) (layer "B.Cu") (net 17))
 (segment (start 110.75 110.25) (end 127 110.25) (width 1) (layer "B.Cu") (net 17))
 (segment (start 133.58 92.92) (end 134.38 92.92) (width 1) (layer "B.Cu") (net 17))
 (segment (start 128 106) (end 132 102) (width 1) (layer "B.Cu") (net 17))
 (segment (start 108.5 108) (end 110.75 110.25) (width 1) (layer "B.Cu") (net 17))
 (segment (start 127 110.25) (end 128 109.25) (width 1) (layer "B.Cu") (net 17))
 (segment (start 106.25 108) (end 105.5 107.25) (width 1) (layer "B.Cu") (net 17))
 (segment (start 99 107.25) (end 105.5 107.25) (width 1) (layer "B.Cu") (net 17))
 (segment (start 110.25 121.75) (end 108.5 120) (width 1) (layer "B.Cu") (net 5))
 (segment (start 134.38 108.16) (end 133.965 108.16) (width 1) (layer "B.Cu") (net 5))
 (segment (start 132 117.25) (end 127.5 121.75) (width 1) (layer "B.Cu") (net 5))
 (segment (start 127.5 121.75) (end 110.25 121.75) (width 1) (layer "B.Cu") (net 5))
 (segment (start 108.5 120) (end 106.25 120) (width 1) (layer "B.Cu") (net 5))
 (segment (start 99 119.25) (end 105.5 119.25) (width 1) (layer "B.Cu") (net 5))
 (segment (start 132 110.125) (end 132 117.25) (width 1) (layer "B.Cu") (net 5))
 (segment (start 133.965 108.16) (end 132 110.125) (width 1) (layer "B.Cu") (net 5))
 (segment (start 106.25 120) (end 105.5 119.25) (width 1) (layer "B.Cu") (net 5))
 (segment (start 110.25 133) (end 128.25 133) (width 1) (layer "B.Cu") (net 9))
 (segment (start 135.49 113.24) (end 134.38 113.24) (width 1) (layer "B.Cu") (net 9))
 (segment (start 99 130.5) (end 105.5 130.5) (width 1) (layer "B.Cu") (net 9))
 (segment (start 106.25 131.25) (end 105.5 130.5) (width 1) (layer "B.Cu") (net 9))
 (segment (start 137 114.75) (end 135.49 113.24) (width 1) (layer "B.Cu") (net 9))
 (segment (start 108.5 131.25) (end 110.25 133) (width 1) (layer "B.Cu") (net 9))
 (segment (start 128.25 133) (end 137 124.25) (width 1) (layer "B.Cu") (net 9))
 (segment (start 137 124.25) (end 137 114.75) (width 1) (layer "B.Cu") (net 9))
 (segment (start 108.5 131.25) (end 106.25 131.25) (width 1) (layer "B.Cu") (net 9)))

